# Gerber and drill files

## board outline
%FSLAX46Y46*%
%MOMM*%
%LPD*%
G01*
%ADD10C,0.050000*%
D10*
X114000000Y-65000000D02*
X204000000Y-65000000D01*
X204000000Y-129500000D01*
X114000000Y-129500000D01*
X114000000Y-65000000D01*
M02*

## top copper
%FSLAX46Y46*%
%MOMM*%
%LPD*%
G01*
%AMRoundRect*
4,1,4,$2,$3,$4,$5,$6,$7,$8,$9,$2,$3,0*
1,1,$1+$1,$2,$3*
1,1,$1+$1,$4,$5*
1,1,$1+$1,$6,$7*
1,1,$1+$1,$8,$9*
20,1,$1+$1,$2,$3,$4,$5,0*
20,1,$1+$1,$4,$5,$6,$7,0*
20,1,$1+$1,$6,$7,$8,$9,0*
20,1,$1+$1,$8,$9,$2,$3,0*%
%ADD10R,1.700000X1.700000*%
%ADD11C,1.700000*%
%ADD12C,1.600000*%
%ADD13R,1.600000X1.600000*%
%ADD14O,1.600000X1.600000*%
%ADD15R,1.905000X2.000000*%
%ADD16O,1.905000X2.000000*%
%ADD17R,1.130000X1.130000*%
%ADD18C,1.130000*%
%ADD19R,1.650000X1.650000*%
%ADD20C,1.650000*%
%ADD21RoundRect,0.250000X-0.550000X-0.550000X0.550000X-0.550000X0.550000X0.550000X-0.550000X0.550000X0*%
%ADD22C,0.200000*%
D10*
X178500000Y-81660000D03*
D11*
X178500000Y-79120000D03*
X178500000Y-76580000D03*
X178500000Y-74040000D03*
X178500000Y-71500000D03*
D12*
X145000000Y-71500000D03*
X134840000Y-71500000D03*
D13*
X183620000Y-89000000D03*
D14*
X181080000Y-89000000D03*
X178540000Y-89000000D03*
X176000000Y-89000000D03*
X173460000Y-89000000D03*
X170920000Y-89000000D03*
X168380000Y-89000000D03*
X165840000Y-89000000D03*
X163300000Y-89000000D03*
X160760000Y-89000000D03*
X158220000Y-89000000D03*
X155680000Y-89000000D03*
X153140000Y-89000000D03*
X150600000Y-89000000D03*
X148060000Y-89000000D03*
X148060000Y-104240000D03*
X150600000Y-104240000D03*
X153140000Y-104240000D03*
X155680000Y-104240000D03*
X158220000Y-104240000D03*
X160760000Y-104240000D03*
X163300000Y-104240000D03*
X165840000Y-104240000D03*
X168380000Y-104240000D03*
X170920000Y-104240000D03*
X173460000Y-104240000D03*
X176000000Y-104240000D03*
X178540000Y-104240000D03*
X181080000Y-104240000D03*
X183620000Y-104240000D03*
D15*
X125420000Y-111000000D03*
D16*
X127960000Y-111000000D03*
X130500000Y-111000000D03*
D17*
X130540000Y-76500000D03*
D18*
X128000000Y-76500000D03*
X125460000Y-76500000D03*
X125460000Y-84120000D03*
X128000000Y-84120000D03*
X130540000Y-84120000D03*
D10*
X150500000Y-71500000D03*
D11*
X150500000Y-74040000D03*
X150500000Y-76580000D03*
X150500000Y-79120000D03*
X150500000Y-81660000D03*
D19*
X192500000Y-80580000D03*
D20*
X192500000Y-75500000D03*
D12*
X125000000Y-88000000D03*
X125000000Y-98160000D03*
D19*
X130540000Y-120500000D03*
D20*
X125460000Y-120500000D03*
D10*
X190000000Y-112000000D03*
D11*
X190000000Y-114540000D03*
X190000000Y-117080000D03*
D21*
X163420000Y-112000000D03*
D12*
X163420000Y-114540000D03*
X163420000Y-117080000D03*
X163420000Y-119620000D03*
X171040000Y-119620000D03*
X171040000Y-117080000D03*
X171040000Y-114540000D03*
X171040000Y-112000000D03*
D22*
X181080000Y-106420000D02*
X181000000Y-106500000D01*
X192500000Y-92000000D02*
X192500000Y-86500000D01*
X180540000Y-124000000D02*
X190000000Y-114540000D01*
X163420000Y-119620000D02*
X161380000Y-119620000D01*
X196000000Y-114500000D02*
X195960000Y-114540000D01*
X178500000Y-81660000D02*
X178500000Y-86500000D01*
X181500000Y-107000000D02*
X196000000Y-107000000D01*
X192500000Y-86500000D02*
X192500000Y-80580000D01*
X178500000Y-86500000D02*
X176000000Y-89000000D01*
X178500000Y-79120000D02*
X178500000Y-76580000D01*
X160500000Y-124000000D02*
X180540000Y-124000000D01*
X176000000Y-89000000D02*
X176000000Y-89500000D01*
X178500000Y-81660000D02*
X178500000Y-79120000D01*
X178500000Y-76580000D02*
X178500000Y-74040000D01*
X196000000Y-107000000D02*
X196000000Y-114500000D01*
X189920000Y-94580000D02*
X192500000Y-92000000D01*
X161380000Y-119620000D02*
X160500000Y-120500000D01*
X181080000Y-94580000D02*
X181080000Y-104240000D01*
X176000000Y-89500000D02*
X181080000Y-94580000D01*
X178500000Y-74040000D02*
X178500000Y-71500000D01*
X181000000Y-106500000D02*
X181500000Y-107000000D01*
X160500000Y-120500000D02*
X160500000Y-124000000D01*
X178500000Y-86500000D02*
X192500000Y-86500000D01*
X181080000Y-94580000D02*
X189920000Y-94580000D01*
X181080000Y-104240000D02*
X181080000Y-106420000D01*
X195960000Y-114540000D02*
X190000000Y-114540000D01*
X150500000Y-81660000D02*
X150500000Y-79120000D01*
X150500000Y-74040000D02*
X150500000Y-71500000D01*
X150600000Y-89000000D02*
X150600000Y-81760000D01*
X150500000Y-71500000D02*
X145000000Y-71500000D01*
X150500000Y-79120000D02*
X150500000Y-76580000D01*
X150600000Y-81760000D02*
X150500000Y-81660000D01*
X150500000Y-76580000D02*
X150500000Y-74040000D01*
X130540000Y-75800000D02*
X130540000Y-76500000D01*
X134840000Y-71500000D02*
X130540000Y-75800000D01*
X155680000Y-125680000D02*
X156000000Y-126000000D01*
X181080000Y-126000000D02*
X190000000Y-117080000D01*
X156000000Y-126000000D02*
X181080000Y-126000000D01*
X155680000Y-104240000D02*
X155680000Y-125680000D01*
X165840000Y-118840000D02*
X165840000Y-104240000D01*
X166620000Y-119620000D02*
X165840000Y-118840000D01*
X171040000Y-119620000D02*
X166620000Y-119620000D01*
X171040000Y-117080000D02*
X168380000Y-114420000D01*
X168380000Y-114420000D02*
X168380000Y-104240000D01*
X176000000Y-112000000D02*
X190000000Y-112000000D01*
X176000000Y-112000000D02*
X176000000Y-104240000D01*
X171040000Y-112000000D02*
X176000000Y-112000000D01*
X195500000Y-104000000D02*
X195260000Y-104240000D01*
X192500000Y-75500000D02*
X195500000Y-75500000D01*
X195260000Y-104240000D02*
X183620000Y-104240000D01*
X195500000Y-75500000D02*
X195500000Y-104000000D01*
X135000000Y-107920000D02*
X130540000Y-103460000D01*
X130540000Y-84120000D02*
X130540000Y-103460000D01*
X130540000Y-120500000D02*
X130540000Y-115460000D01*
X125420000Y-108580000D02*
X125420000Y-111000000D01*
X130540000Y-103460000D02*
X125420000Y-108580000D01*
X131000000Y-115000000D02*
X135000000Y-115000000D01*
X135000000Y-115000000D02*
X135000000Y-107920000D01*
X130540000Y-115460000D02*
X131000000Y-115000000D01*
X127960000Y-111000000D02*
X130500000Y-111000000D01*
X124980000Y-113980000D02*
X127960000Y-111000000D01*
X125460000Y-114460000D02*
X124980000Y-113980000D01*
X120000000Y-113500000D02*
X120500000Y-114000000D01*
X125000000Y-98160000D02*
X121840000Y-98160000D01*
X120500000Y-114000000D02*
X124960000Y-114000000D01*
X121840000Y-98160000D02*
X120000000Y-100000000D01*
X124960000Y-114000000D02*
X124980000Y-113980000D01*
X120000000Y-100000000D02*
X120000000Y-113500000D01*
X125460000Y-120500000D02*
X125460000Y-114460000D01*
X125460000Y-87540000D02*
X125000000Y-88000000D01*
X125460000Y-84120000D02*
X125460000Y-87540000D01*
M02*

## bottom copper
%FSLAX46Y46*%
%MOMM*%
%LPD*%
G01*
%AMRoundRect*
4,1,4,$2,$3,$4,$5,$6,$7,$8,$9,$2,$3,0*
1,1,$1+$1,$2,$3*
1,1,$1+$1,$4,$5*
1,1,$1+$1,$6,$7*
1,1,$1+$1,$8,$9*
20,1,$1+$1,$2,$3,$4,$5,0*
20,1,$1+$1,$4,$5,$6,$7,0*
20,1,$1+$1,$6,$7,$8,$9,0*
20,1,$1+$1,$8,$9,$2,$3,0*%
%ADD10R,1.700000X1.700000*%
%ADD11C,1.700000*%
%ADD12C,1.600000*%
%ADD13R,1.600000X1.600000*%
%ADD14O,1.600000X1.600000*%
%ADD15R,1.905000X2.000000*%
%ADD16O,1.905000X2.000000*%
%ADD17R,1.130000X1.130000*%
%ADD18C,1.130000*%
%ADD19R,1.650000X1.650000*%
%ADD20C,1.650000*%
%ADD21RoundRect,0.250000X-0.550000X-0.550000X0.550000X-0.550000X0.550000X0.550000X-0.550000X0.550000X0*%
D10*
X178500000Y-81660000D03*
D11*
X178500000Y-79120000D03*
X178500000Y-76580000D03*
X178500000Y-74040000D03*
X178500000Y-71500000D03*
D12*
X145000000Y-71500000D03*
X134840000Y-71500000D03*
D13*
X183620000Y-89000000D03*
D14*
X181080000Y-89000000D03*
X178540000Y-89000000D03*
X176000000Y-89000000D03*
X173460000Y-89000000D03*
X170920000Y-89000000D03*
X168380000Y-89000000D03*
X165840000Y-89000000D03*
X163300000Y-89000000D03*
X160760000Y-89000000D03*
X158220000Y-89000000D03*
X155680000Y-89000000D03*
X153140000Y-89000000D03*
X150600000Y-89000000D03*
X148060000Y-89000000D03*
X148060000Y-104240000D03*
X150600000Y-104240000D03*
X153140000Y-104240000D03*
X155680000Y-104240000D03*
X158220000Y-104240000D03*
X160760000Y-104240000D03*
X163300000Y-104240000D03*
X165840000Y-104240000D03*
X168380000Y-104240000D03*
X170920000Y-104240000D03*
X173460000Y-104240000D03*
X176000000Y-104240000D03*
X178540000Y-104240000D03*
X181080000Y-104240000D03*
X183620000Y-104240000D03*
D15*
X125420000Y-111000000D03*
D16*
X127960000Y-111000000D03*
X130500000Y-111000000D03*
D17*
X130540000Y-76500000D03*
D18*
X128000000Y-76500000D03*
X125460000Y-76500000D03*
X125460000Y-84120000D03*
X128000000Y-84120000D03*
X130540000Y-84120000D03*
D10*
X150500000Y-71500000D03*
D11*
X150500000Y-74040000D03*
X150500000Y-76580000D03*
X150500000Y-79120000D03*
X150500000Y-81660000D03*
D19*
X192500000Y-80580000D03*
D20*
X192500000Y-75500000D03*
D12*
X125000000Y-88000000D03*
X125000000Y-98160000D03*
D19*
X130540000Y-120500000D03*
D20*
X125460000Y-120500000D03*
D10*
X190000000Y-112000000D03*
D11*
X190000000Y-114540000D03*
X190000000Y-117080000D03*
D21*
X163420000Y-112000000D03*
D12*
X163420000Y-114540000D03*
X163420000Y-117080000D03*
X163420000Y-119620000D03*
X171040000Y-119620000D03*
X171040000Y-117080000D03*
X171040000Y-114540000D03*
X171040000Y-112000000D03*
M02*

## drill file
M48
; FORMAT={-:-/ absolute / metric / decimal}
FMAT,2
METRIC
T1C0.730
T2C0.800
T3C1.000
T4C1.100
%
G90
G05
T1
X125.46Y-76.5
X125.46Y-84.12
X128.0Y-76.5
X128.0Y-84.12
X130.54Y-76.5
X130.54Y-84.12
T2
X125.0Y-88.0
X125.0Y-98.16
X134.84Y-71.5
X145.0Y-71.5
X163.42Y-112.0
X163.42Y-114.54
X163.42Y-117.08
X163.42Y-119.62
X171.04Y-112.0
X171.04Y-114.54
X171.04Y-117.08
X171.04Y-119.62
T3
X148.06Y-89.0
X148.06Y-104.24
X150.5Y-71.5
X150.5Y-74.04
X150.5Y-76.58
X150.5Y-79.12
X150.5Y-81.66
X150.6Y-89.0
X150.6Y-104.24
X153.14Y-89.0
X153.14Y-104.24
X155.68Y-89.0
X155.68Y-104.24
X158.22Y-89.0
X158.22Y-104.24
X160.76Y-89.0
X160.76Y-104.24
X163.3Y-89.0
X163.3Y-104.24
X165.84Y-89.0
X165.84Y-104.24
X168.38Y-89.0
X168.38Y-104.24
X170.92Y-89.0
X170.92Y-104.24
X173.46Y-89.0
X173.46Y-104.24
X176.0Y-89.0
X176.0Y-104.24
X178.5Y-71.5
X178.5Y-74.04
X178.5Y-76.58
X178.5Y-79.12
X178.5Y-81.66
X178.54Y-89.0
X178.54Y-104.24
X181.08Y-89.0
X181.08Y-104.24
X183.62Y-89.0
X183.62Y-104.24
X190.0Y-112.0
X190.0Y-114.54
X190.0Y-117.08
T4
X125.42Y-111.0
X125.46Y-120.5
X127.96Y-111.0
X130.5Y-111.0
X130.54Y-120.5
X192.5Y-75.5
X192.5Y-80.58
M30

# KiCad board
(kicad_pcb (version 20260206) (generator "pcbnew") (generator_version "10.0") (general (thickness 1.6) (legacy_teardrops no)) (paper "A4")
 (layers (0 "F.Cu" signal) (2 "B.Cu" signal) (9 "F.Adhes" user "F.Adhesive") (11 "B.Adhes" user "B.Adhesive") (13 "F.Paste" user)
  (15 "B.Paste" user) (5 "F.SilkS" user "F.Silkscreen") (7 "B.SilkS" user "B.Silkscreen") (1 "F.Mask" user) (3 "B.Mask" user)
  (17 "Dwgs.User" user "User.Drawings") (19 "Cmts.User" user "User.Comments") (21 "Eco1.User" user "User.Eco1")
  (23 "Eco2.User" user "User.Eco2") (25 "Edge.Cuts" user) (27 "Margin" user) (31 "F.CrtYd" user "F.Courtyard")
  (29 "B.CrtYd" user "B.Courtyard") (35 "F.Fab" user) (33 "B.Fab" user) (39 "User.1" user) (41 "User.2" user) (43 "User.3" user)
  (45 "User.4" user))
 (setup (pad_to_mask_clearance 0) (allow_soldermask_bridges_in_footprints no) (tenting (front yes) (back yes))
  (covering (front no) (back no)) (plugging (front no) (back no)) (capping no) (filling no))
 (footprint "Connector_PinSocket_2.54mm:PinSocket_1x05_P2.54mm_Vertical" (layer "F.Cu") (at 178.5 81.66 180)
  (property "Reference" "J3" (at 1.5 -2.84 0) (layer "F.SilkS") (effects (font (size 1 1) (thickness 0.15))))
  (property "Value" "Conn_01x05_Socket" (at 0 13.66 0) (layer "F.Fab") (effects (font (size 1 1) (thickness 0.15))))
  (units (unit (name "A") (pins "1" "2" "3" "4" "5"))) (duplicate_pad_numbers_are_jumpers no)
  (pad "1" thru_hole rect (at 0 0 180) (size 1.7 1.7) (drill 1) (layers "*.Cu" "*.Mask") (remove_unused_layers no) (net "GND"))
  (pad "2" thru_hole circle (at 0 2.54 180) (size 1.7 1.7) (drill 1) (layers "*.Cu" "*.Mask") (remove_unused_layers no) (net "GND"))
  (pad "3" thru_hole circle (at 0 5.08 180) (size 1.7 1.7) (drill 1) (layers "*.Cu" "*.Mask") (remove_unused_layers no) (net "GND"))
  (pad "4" thru_hole circle (at 0 7.62 180) (size 1.7 1.7) (drill 1) (layers "*.Cu" "*.Mask") (remove_unused_layers no) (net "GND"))
  (pad "5" thru_hole circle (at 0 10.16 180) (size 1.7 1.7) (drill 1) (layers "*.Cu" "*.Mask") (remove_unused_layers no) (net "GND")))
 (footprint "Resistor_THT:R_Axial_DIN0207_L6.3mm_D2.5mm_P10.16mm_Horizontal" (layer "F.Cu") (at 145 71.5 180)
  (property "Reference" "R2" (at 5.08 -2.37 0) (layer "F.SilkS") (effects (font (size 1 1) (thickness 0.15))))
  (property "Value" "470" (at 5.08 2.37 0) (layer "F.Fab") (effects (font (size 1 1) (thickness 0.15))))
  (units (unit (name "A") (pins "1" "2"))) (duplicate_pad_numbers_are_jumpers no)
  (pad "1" thru_hole circle (at 0 0 180) (size 1.6 1.6) (drill 0.8) (layers "*.Cu" "*.Mask") (remove_unused_layers no) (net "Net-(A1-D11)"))
  (pad "2" thru_hole circle (at 10.16 0 180) (size 1.6 1.6) (drill 0.8) (layers "*.Cu" "*.Mask") (remove_unused_layers no)
   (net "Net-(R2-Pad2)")))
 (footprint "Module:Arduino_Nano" (layer "F.Cu") (at 183.62 89 -90)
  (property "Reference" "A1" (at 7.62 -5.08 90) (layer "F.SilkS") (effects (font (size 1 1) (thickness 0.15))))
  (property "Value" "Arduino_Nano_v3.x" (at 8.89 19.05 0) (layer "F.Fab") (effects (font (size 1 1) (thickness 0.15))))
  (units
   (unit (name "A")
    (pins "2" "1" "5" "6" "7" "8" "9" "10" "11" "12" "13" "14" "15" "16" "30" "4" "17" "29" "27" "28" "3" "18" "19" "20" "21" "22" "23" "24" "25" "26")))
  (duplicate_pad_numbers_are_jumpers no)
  (pad "1" thru_hole rect (at 0 0 270) (size 1.6 1.6) (drill 1) (layers "*.Cu" "*.Mask") (remove_unused_layers no)
   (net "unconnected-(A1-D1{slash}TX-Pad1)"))
  (pad "2" thru_hole oval (at 0 2.54 270) (size 1.6 1.6) (drill 1) (layers "*.Cu" "*.Mask") (remove_unused_layers no)
   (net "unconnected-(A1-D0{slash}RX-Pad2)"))
  (pad "3" thru_hole oval (at 0 5.08 270) (size 1.6 1.6) (drill 1) (layers "*.Cu" "*.Mask") (remove_unused_layers no)
   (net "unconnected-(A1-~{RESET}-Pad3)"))
  (pad "4" thru_hole oval (at 0 7.62 270) (size 1.6 1.6) (drill 1) (layers "*.Cu" "*.Mask") (remove_unused_layers no) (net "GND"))
  (pad "5" thru_hole oval (at 0 10.16 270) (size 1.6 1.6) (drill 1) (layers "*.Cu" "*.Mask") (remove_unused_layers no)
   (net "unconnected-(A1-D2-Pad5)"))
  (pad "6" thru_hole oval (at 0 12.7 270) (size 1.6 1.6) (drill 1) (layers "*.Cu" "*.Mask") (remove_unused_layers no)
   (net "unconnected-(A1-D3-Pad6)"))
  (pad "7" thru_hole oval (at 0 15.24 270) (size 1.6 1.6) (drill 1) (layers "*.Cu" "*.Mask") (remove_unused_layers no)
   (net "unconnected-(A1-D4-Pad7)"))
  (pad "8" thru_hole oval (at 0 17.78 270) (size 1.6 1.6) (drill 1) (layers "*.Cu" "*.Mask") (remove_unused_layers no)
   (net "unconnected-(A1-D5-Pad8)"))
  (pad "9" thru_hole oval (at 0 20.32 270) (size 1.6 1.6) (drill 1) (layers "*.Cu" "*.Mask") (remove_unused_layers no)
   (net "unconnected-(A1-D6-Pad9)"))
  (pad "10" thru_hole oval (at 0 22.86 270) (size 1.6 1.6) (drill 1) (layers "*.Cu" "*.Mask") (remove_unused_layers no)
   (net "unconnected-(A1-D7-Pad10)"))
  (pad "11" thru_hole oval (at 0 25.4 270) (size 1.6 1.6) (drill 1) (layers "*.Cu" "*.Mask") (remove_unused_layers no)
   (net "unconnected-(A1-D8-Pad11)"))
  (pad "12" thru_hole oval (at 0 27.94 270) (size 1.6 1.6) (drill 1) (layers "*.Cu" "*.Mask") (remove_unused_layers no)
   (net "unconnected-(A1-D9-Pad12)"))
  (pad "13" thru_hole oval (at 0 30.48 270) (size 1.6 1.6) (drill 1) (layers "*.Cu" "*.Mask") (remove_unused_layers no)
   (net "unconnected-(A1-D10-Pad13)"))
  (pad "14" thru_hole oval (at 0 33.02 270) (size 1.6 1.6) (drill 1) (layers "*.Cu" "*.Mask") (remove_unused_layers no) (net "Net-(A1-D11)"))
  (pad "15" thru_hole oval (at 0 35.56 270) (size 1.6 1.6) (drill 1) (layers "*.Cu" "*.Mask") (remove_unused_layers no)
   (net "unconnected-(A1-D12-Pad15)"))
  (pad "16" thru_hole oval (at 15.24 35.56 270) (size 1.6 1.6) (drill 1) (layers "*.Cu" "*.Mask") (remove_unused_layers no)
   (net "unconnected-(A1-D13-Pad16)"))
  (pad "17" thru_hole oval (at 15.24 33.02 270) (size 1.6 1.6) (drill 1) (layers "*.Cu" "*.Mask") (remove_unused_layers no)
   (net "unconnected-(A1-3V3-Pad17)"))
  (pad "18" thru_hole oval (at 15.24 30.48 270) (size 1.6 1.6) (drill 1) (layers "*.Cu" "*.Mask") (remove_unused_layers no)
   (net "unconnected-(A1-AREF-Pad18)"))
  (pad "19" thru_hole oval (at 15.24 27.94 270) (size 1.6 1.6) (drill 1) (layers "*.Cu" "*.Mask") (remove_unused_layers no)
   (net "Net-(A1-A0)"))
  (pad "20" thru_hole oval (at 15.24 25.4 270) (size 1.6 1.6) (drill 1) (layers "*.Cu" "*.Mask") (remove_unused_layers no)
   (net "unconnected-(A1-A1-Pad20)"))
  (pad "21" thru_hole oval (at 15.24 22.86 270) (size 1.6 1.6) (drill 1) (layers "*.Cu" "*.Mask") (remove_unused_layers no)
   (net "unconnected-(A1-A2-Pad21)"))
  (pad "22" thru_hole oval (at 15.24 20.32 270) (size 1.6 1.6) (drill 1) (layers "*.Cu" "*.Mask") (remove_unused_layers no)
   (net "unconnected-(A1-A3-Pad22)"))
  (pad "23" thru_hole oval (at 15.24 17.78 270) (size 1.6 1.6) (drill 1) (layers "*.Cu" "*.Mask") (remove_unused_layers no)
   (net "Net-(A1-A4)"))
  (pad "24" thru_hole oval (at 15.24 15.24 270) (size 1.6 1.6) (drill 1) (layers "*.Cu" "*.Mask") (remove_unused_layers no)
   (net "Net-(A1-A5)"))
  (pad "25" thru_hole oval (at 15.24 12.7 270) (size 1.6 1.6) (drill 1) (layers "*.Cu" "*.Mask") (remove_unused_layers no)
   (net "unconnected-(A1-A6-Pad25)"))
  (pad "26" thru_hole oval (at 15.24 10.16 270) (size 1.6 1.6) (drill 1) (layers "*.Cu" "*.Mask") (remove_unused_layers no)
   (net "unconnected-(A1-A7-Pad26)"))
  (pad "27" thru_hole oval (at 15.24 7.62 270) (size 1.6 1.6) (drill 1) (layers "*.Cu" "*.Mask") (remove_unused_layers no)
   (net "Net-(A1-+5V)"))
  (pad "28" thru_hole oval (at 15.24 5.08 270) (size 1.6 1.6) (drill 1) (layers "*.Cu" "*.Mask") (remove_unused_layers no)
   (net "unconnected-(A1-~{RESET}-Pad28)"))
  (pad "29" thru_hole oval (at 15.24 2.54 270) (size 1.6 1.6) (drill 1) (layers "*.Cu" "*.Mask") (remove_unused_layers no) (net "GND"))
  (pad "30" thru_hole oval (at 15.24 0 270) (size 1.6 1.6) (drill 1) (layers "*.Cu" "*.Mask") (remove_unused_layers no) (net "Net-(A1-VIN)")))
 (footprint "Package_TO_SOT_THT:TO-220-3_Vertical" (layer "F.Cu") (at 125.42 111)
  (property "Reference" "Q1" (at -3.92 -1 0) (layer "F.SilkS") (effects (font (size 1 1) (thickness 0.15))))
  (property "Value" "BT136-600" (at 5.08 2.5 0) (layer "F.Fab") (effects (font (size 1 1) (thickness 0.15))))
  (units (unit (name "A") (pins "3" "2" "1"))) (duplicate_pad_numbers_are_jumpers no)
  (pad "1" thru_hole rect (at 0 0) (size 1.905 2) (drill 1.1) (layers "*.Cu" "*.Mask") (remove_unused_layers no) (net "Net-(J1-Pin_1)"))
  (pad "2" thru_hole oval (at 2.54 0) (size 1.905 2) (drill 1.1) (layers "*.Cu" "*.Mask") (remove_unused_layers no) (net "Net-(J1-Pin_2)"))
  (pad "3" thru_hole oval (at 5.08 0) (size 1.905 2) (drill 1.1) (layers "*.Cu" "*.Mask") (remove_unused_layers no) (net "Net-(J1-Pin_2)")))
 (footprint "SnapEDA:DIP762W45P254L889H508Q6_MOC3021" (layer "F.Cu") (at 128 80.31 -90)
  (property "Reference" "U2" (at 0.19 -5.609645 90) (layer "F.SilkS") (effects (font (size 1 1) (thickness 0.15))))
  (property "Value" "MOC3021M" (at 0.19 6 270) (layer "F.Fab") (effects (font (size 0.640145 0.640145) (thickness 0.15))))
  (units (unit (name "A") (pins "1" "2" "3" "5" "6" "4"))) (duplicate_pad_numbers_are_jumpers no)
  (pad "1" thru_hole rect (at -3.81 -2.54 270) (size 1.13 1.13) (drill 0.73) (layers "*.Cu" "*.Mask") (remove_unused_layers no)
   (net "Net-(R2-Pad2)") (solder_mask_margin 0.102))
  (pad "2" thru_hole circle (at -3.81 0 270) (size 1.13 1.13) (drill 0.73) (layers "*.Cu" "*.Mask") (remove_unused_layers no)
   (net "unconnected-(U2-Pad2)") (solder_mask_margin 0.102))
  (pad "3" thru_hole circle (at -3.81 2.54 270) (size 1.13 1.13) (drill 0.73) (layers "*.Cu" "*.Mask") (remove_unused_layers no)
   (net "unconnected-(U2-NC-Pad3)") (solder_mask_margin 0.102))
  (pad "4" thru_hole circle (at 3.81 2.54 270) (size 1.13 1.13) (drill 0.73) (layers "*.Cu" "*.Mask") (remove_unused_layers no)
   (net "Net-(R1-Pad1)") (solder_mask_margin 0.102))
  (pad "5" thru_hole circle (at 3.81 0 270) (size 1.13 1.13) (drill 0.73) (layers "*.Cu" "*.Mask") (remove_unused_layers no)
   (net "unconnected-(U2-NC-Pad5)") (solder_mask_margin 0.102))
  (pad "6" thru_hole circle (at 3.81 -2.54 270) (size 1.13 1.13) (drill 0.73) (layers "*.Cu" "*.Mask") (remove_unused_layers no)
   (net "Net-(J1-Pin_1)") (solder_mask_margin 0.102)))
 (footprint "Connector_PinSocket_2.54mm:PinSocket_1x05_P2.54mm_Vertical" (layer "F.Cu") (at 150.5 71.5)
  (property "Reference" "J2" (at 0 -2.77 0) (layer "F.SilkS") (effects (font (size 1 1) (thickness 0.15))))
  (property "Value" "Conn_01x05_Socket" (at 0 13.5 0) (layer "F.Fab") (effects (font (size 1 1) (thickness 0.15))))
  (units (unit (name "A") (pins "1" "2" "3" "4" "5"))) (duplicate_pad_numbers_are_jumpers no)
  (pad "1" thru_hole rect (at 0 0) (size 1.7 1.7) (drill 1) (layers "*.Cu" "*.Mask") (remove_unused_layers no) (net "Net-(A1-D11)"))
  (pad "2" thru_hole circle (at 0 2.54) (size 1.7 1.7) (drill 1) (layers "*.Cu" "*.Mask") (remove_unused_layers no) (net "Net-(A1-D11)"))
  (pad "3" thru_hole circle (at 0 5.08) (size 1.7 1.7) (drill 1) (layers "*.Cu" "*.Mask") (remove_unused_layers no) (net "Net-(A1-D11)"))
  (pad "4" thru_hole circle (at 0 7.62) (size 1.7 1.7) (drill 1) (layers "*.Cu" "*.Mask") (remove_unused_layers no) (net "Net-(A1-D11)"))
  (pad "5" thru_hole circle (at 0 10.16) (size 1.7 1.7) (drill 1) (layers "*.Cu" "*.Mask") (remove_unused_layers no) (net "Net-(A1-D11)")))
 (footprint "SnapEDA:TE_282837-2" (layer "F.Cu") (at 192.5 78.04 90)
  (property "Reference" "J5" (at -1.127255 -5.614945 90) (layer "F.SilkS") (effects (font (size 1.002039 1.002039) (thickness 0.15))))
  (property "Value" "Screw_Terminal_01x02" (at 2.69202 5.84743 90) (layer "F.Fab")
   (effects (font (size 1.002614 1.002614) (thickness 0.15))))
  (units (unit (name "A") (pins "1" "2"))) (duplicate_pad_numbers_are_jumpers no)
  (pad "1" thru_hole rect (at -2.54 0 90) (size 1.65 1.65) (drill 1.1) (layers "*.Cu" "*.Mask") (remove_unused_layers no) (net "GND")
   (solder_mask_margin 0.102))
  (pad "2" thru_hole circle (at 2.54 0 90) (size 1.65 1.65) (drill 1.1) (layers "*.Cu" "*.Mask") (remove_unused_layers no)
   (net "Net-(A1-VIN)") (solder_mask_margin 0.102)))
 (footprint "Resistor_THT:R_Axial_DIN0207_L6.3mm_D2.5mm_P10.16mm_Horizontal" (layer "F.Cu") (at 125 88 -90)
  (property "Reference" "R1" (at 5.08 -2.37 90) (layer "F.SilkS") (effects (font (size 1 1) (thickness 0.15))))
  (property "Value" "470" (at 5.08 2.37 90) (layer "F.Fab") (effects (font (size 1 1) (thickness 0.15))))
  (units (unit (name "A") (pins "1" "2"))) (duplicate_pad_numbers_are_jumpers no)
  (pad "1" thru_hole circle (at 0 0 270) (size 1.6 1.6) (drill 0.8) (layers "*.Cu" "*.Mask") (remove_unused_layers no) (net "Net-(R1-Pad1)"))
  (pad "2" thru_hole circle (at 10.16 0 270) (size 1.6 1.6) (drill 0.8) (layers "*.Cu" "*.Mask") (remove_unused_layers no)
   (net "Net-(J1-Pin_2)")))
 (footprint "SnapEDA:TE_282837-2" (layer "F.Cu") (at 128 120.5 180)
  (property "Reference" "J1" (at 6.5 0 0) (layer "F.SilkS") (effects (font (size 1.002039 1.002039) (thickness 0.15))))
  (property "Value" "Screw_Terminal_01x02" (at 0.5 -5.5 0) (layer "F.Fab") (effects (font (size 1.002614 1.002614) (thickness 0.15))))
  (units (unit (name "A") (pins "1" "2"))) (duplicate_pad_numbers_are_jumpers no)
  (pad "1" thru_hole rect (at -2.54 0 180) (size 1.65 1.65) (drill 1.1) (layers "*.Cu" "*.Mask") (remove_unused_layers no)
   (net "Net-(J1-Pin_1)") (solder_mask_margin 0.102))
  (pad "2" thru_hole circle (at 2.54 0 180) (size 1.65 1.65) (drill 1.1) (layers "*.Cu" "*.Mask") (remove_unused_layers no)
   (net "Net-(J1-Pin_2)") (solder_mask_margin 0.102)))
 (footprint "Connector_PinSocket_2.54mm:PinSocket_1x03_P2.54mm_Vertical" (layer "F.Cu") (at 190 112)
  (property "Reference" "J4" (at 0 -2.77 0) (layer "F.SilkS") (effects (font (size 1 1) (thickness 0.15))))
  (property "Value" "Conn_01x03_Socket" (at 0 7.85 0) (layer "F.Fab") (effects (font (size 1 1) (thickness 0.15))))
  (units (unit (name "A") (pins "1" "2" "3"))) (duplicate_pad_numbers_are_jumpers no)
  (pad "1" thru_hole rect (at 0 0) (size 1.7 1.7) (drill 1) (layers "*.Cu" "*.Mask") (remove_unused_layers no) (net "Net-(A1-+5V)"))
  (pad "2" thru_hole circle (at 0 2.54) (size 1.7 1.7) (drill 1) (layers "*.Cu" "*.Mask") (remove_unused_layers no) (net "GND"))
  (pad "3" thru_hole circle (at 0 5.08) (size 1.7 1.7) (drill 1) (layers "*.Cu" "*.Mask") (remove_unused_layers no) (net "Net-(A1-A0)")))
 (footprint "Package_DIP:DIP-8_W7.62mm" (layer "F.Cu") (at 163.42 112)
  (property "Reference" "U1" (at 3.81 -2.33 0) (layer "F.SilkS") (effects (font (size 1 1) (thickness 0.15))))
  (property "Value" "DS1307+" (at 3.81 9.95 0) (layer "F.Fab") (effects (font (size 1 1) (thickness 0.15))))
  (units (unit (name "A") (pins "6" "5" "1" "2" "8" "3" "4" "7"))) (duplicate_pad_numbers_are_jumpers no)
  (pad "1" thru_hole roundrect (at 0 0) (size 1.6 1.6) (drill 0.8) (layers "*.Cu" "*.Mask") (remove_unused_layers no)
   (roundrect_rratio 0.15625) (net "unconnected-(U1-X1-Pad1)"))
  (pad "2" thru_hole circle (at 0 2.54) (size 1.6 1.6) (drill 0.8) (layers "*.Cu" "*.Mask") (remove_unused_layers no)
   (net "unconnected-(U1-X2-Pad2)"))
  (pad "3" thru_hole circle (at 0 5.08) (size 1.6 1.6) (drill 0.8) (layers "*.Cu" "*.Mask") (remove_unused_layers no)
   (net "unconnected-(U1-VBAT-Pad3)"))
  (pad "4" thru_hole circle (at 0 7.62) (size 1.6 1.6) (drill 0.8) (layers "*.Cu" "*.Mask") (remove_unused_layers no) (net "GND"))
  (pad "5" thru_hole circle (at 7.62 7.62) (size 1.6 1.6) (drill 0.8) (layers "*.Cu" "*.Mask") (remove_unused_layers no) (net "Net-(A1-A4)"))
  (pad "6" thru_hole circle (at 7.62 5.08) (size 1.6 1.6) (drill 0.8) (layers "*.Cu" "*.Mask") (remove_unused_layers no) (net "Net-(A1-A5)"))
  (pad "7" thru_hole circle (at 7.62 2.54) (size 1.6 1.6) (drill 0.8) (layers "*.Cu" "*.Mask") (remove_unused_layers no)
   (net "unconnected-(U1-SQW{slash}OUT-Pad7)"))
  (pad "8" thru_hole circle (at 7.62 0) (size 1.6 1.6) (drill 0.8) (layers "*.Cu" "*.Mask") (remove_unused_layers no) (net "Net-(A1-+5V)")))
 (gr_rect (start 114 65) (end 204 129.5) (stroke (width 0.05) (type default)) (fill no) (layer "Edge.Cuts"))
 (segment (start 181.08 106.42) (end 181 106.5) (width 0.2) (layer "F.Cu") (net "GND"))
 (segment (start 192.5 92) (end 192.5 86.5) (width 0.2) (layer "F.Cu") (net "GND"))
 (segment (start 180.54 124) (end 190 114.54) (width 0.2) (layer "F.Cu") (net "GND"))
 (segment (start 163.42 119.62) (end 161.38 119.62) (width 0.2) (layer "F.Cu") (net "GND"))
 (segment (start 196 114.5) (end 195.96 114.54) (width 0.2) (layer "F.Cu") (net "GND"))
 (segment (start 178.5 81.66) (end 178.5 86.5) (width 0.2) (layer "F.Cu") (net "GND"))
 (segment (start 181.5 107) (end 196 107) (width 0.2) (layer "F.Cu") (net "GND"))
 (segment (start 192.5 86.5) (end 192.5 80.58) (width 0.2) (layer "F.Cu") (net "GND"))
 (segment (start 178.5 86.5) (end 176 89) (width 0.2) (layer "F.Cu") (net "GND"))
 (segment (start 178.5 79.12) (end 178.5 76.58) (width 0.2) (layer "F.Cu") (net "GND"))
 (segment (start 160.5 124) (end 180.54 124) (width 0.2) (layer "F.Cu") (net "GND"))
 (segment (start 176 89) (end 176 89.5) (width 0.2) (layer "F.Cu") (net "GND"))
 (segment (start 178.5 81.66) (end 178.5 79.12) (width 0.2) (layer "F.Cu") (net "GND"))
 (segment (start 178.5 76.58) (end 178.5 74.04) (width 0.2) (layer "F.Cu") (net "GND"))
 (segment (start 196 107) (end 196 114.5) (width 0.2) (layer "F.Cu") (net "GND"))
 (segment (start 189.92 94.58) (end 192.5 92) (width 0.2) (layer "F.Cu") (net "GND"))
 (segment (start 161.38 119.62) (end 160.5 120.5) (width 0.2) (layer "F.Cu") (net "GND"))
 (segment (start 181.08 94.58) (end 181.08 104.24) (width 0.2) (layer "F.Cu") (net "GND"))
 (segment (start 176 89.5) (end 181.08 94.58) (width 0.2) (layer "F.Cu") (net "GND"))
 (segment (start 178.5 74.04) (end 178.5 71.5) (width 0.2) (layer "F.Cu") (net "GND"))
 (segment (start 181 106.5) (end 181.5 107) (width 0.2) (layer "F.Cu") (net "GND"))
 (segment (start 160.5 120.5) (end 160.5 124) (width 0.2) (layer "F.Cu") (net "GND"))
 (segment (start 178.5 86.5) (end 192.5 86.5) (width 0.2) (layer "F.Cu") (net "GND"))
 (segment (start 181.08 94.58) (end 189.92 94.58) (width 0.2) (layer "F.Cu") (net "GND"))
 (segment (start 181.08 104.24) (end 181.08 106.42) (width 0.2) (layer "F.Cu") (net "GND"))
 (segment (start 195.96 114.54) (end 190 114.54) (width 0.2) (layer "F.Cu") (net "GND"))
 (segment (start 150.5 81.66) (end 150.5 79.12) (width 0.2) (layer "F.Cu") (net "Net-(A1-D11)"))
 (segment (start 150.5 74.04) (end 150.5 71.5) (width 0.2) (layer "F.Cu") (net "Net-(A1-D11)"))
 (segment (start 150.6 89) (end 150.6 81.76) (width 0.2) (layer "F.Cu") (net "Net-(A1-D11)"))
 (segment (start 150.5 71.5) (end 145 71.5) (width 0.2) (layer "F.Cu") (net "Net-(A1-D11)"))
 (segment (start 150.5 79.12) (end 150.5 76.58) (width 0.2) (layer "F.Cu") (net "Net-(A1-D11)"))
 (segment (start 150.6 81.76) (end 150.5 81.66) (width 0.2) (layer "F.Cu") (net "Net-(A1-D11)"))
 (segment (start 150.5 76.58) (end 150.5 74.04) (width 0.2) (layer "F.Cu") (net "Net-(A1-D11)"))
 (segment (start 130.54 75.8) (end 130.54 76.5) (width 0.2) (layer "F.Cu") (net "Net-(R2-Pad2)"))
 (segment (start 134.84 71.5) (end 130.54 75.8) (width 0.2) (layer "F.Cu") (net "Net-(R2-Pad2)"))
 (segment (start 155.68 125.68) (end 156 126) (width 0.2) (layer "F.Cu") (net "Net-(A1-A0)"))
 (segment (start 181.08 126) (end 190 117.08) (width 0.2) (layer "F.Cu") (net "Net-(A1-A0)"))
 (segment (start 156 126) (end 181.08 126) (width 0.2) (layer "F.Cu") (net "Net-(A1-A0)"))
 (segment (start 155.68 104.24) (end 155.68 125.68) (width 0.2) (layer "F.Cu") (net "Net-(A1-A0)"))
 (segment (start 165.84 118.84) (end 165.84 104.24) (width 0.2) (layer "F.Cu") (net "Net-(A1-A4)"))
 (segment (start 166.62 119.62) (end 165.84 118.84) (width 0.2) (layer "F.Cu") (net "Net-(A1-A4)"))
 (segment (start 171.04 119.62) (end 166.62 119.62) (width 0.2) (layer "F.Cu") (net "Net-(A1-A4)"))
 (segment (start 171.04 117.08) (end 168.38 114.42) (width 0.2) (layer "F.Cu") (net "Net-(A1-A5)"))
 (segment (start 168.38 114.42) (end 168.38 104.24) (width 0.2) (layer "F.Cu") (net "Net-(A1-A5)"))
 (segment (start 176 112) (end 190 112) (width 0.2) (layer "F.Cu") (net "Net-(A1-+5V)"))
 (segment (start 176 112) (end 176 104.24) (width 0.2) (layer "F.Cu") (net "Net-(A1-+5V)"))
 (segment (start 171.04 112) (end 176 112) (width 0.2) (layer "F.Cu") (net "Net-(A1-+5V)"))
 (segment (start 195.5 104) (end 195.26 104.24) (width 0.2) (layer "F.Cu") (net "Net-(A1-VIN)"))
 (segment (start 192.5 75.5) (end 195.5 75.5) (width 0.2) (layer "F.Cu") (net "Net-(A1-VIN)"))
 (segment (start 195.26 104.24) (end 183.62 104.24) (width 0.2) (layer "F.Cu") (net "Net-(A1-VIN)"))
 (segment (start 195.5 75.5) (end 195.5 104) (width 0.2) (layer "F.Cu") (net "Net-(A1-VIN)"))
 (segment (start 135 107.92) (end 130.54 103.46) (width 0.2) (layer "F.Cu") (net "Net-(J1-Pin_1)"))
 (segment (start 130.54 84.12) (end 130.54 103.46) (width 0.2) (layer "F.Cu") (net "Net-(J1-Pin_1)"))
 (segment (start 130.54 120.5) (end 130.54 115.46) (width 0.2) (layer "F.Cu") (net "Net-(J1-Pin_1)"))
 (segment (start 125.42 108.58) (end 125.42 111) (width 0.2) (layer "F.Cu") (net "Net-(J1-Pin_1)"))
 (segment (start 130.54 103.46) (end 125.42 108.58) (width 0.2) (layer "F.Cu") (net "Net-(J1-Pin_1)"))
 (segment (start 131 115) (end 135 115) (width 0.2) (layer "F.Cu") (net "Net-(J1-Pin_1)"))
 (segment (start 135 115) (end 135 107.92) (width 0.2) (layer "F.Cu") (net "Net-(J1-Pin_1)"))
 (segment (start 130.54 115.46) (end 131 115) (width 0.2) (layer "F.Cu") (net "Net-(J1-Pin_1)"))
 (segment (start 127.96 111) (end 130.5 111) (width 0.2) (layer "F.Cu") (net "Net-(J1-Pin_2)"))
 (segment (start 124.98 113.98) (end 127.96 111) (width 0.2) (layer "F.Cu") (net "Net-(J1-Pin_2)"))
 (segment (start 125.46 114.46) (end 124.98 113.98) (width 0.2) (layer "F.Cu") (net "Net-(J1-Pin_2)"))
 (segment (start 120 113.5) (end 120.5 114) (width 0.2) (layer "F.Cu") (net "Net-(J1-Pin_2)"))
 (segment (start 125 98.16) (end 121.84 98.16) (width 0.2) (layer "F.Cu") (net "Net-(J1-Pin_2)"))
 (segment (start 120.5 114) (end 124.96 114) (width 0.2) (layer "F.Cu") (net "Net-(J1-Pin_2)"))
 (segment (start 121.84 98.16) (end 120 100) (width 0.2) (layer "F.Cu") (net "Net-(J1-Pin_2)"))
 (segment (start 124.96 114) (end 124.98 113.98) (width 0.2) (layer "F.Cu") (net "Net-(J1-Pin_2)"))
 (segment (start 120 100) (end 120 113.5) (width 0.2) (layer "F.Cu") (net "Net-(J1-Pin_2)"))
 (segment (start 125.46 120.5) (end 125.46 114.46) (width 0.2) (layer "F.Cu") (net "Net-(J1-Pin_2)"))
 (segment (start 125.46 87.54) (end 125 88) (width 0.2) (layer "F.Cu") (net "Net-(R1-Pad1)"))
 (segment (start 125.46 84.12) (end 125.46 87.54) (width 0.2) (layer "F.Cu") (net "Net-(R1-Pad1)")))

